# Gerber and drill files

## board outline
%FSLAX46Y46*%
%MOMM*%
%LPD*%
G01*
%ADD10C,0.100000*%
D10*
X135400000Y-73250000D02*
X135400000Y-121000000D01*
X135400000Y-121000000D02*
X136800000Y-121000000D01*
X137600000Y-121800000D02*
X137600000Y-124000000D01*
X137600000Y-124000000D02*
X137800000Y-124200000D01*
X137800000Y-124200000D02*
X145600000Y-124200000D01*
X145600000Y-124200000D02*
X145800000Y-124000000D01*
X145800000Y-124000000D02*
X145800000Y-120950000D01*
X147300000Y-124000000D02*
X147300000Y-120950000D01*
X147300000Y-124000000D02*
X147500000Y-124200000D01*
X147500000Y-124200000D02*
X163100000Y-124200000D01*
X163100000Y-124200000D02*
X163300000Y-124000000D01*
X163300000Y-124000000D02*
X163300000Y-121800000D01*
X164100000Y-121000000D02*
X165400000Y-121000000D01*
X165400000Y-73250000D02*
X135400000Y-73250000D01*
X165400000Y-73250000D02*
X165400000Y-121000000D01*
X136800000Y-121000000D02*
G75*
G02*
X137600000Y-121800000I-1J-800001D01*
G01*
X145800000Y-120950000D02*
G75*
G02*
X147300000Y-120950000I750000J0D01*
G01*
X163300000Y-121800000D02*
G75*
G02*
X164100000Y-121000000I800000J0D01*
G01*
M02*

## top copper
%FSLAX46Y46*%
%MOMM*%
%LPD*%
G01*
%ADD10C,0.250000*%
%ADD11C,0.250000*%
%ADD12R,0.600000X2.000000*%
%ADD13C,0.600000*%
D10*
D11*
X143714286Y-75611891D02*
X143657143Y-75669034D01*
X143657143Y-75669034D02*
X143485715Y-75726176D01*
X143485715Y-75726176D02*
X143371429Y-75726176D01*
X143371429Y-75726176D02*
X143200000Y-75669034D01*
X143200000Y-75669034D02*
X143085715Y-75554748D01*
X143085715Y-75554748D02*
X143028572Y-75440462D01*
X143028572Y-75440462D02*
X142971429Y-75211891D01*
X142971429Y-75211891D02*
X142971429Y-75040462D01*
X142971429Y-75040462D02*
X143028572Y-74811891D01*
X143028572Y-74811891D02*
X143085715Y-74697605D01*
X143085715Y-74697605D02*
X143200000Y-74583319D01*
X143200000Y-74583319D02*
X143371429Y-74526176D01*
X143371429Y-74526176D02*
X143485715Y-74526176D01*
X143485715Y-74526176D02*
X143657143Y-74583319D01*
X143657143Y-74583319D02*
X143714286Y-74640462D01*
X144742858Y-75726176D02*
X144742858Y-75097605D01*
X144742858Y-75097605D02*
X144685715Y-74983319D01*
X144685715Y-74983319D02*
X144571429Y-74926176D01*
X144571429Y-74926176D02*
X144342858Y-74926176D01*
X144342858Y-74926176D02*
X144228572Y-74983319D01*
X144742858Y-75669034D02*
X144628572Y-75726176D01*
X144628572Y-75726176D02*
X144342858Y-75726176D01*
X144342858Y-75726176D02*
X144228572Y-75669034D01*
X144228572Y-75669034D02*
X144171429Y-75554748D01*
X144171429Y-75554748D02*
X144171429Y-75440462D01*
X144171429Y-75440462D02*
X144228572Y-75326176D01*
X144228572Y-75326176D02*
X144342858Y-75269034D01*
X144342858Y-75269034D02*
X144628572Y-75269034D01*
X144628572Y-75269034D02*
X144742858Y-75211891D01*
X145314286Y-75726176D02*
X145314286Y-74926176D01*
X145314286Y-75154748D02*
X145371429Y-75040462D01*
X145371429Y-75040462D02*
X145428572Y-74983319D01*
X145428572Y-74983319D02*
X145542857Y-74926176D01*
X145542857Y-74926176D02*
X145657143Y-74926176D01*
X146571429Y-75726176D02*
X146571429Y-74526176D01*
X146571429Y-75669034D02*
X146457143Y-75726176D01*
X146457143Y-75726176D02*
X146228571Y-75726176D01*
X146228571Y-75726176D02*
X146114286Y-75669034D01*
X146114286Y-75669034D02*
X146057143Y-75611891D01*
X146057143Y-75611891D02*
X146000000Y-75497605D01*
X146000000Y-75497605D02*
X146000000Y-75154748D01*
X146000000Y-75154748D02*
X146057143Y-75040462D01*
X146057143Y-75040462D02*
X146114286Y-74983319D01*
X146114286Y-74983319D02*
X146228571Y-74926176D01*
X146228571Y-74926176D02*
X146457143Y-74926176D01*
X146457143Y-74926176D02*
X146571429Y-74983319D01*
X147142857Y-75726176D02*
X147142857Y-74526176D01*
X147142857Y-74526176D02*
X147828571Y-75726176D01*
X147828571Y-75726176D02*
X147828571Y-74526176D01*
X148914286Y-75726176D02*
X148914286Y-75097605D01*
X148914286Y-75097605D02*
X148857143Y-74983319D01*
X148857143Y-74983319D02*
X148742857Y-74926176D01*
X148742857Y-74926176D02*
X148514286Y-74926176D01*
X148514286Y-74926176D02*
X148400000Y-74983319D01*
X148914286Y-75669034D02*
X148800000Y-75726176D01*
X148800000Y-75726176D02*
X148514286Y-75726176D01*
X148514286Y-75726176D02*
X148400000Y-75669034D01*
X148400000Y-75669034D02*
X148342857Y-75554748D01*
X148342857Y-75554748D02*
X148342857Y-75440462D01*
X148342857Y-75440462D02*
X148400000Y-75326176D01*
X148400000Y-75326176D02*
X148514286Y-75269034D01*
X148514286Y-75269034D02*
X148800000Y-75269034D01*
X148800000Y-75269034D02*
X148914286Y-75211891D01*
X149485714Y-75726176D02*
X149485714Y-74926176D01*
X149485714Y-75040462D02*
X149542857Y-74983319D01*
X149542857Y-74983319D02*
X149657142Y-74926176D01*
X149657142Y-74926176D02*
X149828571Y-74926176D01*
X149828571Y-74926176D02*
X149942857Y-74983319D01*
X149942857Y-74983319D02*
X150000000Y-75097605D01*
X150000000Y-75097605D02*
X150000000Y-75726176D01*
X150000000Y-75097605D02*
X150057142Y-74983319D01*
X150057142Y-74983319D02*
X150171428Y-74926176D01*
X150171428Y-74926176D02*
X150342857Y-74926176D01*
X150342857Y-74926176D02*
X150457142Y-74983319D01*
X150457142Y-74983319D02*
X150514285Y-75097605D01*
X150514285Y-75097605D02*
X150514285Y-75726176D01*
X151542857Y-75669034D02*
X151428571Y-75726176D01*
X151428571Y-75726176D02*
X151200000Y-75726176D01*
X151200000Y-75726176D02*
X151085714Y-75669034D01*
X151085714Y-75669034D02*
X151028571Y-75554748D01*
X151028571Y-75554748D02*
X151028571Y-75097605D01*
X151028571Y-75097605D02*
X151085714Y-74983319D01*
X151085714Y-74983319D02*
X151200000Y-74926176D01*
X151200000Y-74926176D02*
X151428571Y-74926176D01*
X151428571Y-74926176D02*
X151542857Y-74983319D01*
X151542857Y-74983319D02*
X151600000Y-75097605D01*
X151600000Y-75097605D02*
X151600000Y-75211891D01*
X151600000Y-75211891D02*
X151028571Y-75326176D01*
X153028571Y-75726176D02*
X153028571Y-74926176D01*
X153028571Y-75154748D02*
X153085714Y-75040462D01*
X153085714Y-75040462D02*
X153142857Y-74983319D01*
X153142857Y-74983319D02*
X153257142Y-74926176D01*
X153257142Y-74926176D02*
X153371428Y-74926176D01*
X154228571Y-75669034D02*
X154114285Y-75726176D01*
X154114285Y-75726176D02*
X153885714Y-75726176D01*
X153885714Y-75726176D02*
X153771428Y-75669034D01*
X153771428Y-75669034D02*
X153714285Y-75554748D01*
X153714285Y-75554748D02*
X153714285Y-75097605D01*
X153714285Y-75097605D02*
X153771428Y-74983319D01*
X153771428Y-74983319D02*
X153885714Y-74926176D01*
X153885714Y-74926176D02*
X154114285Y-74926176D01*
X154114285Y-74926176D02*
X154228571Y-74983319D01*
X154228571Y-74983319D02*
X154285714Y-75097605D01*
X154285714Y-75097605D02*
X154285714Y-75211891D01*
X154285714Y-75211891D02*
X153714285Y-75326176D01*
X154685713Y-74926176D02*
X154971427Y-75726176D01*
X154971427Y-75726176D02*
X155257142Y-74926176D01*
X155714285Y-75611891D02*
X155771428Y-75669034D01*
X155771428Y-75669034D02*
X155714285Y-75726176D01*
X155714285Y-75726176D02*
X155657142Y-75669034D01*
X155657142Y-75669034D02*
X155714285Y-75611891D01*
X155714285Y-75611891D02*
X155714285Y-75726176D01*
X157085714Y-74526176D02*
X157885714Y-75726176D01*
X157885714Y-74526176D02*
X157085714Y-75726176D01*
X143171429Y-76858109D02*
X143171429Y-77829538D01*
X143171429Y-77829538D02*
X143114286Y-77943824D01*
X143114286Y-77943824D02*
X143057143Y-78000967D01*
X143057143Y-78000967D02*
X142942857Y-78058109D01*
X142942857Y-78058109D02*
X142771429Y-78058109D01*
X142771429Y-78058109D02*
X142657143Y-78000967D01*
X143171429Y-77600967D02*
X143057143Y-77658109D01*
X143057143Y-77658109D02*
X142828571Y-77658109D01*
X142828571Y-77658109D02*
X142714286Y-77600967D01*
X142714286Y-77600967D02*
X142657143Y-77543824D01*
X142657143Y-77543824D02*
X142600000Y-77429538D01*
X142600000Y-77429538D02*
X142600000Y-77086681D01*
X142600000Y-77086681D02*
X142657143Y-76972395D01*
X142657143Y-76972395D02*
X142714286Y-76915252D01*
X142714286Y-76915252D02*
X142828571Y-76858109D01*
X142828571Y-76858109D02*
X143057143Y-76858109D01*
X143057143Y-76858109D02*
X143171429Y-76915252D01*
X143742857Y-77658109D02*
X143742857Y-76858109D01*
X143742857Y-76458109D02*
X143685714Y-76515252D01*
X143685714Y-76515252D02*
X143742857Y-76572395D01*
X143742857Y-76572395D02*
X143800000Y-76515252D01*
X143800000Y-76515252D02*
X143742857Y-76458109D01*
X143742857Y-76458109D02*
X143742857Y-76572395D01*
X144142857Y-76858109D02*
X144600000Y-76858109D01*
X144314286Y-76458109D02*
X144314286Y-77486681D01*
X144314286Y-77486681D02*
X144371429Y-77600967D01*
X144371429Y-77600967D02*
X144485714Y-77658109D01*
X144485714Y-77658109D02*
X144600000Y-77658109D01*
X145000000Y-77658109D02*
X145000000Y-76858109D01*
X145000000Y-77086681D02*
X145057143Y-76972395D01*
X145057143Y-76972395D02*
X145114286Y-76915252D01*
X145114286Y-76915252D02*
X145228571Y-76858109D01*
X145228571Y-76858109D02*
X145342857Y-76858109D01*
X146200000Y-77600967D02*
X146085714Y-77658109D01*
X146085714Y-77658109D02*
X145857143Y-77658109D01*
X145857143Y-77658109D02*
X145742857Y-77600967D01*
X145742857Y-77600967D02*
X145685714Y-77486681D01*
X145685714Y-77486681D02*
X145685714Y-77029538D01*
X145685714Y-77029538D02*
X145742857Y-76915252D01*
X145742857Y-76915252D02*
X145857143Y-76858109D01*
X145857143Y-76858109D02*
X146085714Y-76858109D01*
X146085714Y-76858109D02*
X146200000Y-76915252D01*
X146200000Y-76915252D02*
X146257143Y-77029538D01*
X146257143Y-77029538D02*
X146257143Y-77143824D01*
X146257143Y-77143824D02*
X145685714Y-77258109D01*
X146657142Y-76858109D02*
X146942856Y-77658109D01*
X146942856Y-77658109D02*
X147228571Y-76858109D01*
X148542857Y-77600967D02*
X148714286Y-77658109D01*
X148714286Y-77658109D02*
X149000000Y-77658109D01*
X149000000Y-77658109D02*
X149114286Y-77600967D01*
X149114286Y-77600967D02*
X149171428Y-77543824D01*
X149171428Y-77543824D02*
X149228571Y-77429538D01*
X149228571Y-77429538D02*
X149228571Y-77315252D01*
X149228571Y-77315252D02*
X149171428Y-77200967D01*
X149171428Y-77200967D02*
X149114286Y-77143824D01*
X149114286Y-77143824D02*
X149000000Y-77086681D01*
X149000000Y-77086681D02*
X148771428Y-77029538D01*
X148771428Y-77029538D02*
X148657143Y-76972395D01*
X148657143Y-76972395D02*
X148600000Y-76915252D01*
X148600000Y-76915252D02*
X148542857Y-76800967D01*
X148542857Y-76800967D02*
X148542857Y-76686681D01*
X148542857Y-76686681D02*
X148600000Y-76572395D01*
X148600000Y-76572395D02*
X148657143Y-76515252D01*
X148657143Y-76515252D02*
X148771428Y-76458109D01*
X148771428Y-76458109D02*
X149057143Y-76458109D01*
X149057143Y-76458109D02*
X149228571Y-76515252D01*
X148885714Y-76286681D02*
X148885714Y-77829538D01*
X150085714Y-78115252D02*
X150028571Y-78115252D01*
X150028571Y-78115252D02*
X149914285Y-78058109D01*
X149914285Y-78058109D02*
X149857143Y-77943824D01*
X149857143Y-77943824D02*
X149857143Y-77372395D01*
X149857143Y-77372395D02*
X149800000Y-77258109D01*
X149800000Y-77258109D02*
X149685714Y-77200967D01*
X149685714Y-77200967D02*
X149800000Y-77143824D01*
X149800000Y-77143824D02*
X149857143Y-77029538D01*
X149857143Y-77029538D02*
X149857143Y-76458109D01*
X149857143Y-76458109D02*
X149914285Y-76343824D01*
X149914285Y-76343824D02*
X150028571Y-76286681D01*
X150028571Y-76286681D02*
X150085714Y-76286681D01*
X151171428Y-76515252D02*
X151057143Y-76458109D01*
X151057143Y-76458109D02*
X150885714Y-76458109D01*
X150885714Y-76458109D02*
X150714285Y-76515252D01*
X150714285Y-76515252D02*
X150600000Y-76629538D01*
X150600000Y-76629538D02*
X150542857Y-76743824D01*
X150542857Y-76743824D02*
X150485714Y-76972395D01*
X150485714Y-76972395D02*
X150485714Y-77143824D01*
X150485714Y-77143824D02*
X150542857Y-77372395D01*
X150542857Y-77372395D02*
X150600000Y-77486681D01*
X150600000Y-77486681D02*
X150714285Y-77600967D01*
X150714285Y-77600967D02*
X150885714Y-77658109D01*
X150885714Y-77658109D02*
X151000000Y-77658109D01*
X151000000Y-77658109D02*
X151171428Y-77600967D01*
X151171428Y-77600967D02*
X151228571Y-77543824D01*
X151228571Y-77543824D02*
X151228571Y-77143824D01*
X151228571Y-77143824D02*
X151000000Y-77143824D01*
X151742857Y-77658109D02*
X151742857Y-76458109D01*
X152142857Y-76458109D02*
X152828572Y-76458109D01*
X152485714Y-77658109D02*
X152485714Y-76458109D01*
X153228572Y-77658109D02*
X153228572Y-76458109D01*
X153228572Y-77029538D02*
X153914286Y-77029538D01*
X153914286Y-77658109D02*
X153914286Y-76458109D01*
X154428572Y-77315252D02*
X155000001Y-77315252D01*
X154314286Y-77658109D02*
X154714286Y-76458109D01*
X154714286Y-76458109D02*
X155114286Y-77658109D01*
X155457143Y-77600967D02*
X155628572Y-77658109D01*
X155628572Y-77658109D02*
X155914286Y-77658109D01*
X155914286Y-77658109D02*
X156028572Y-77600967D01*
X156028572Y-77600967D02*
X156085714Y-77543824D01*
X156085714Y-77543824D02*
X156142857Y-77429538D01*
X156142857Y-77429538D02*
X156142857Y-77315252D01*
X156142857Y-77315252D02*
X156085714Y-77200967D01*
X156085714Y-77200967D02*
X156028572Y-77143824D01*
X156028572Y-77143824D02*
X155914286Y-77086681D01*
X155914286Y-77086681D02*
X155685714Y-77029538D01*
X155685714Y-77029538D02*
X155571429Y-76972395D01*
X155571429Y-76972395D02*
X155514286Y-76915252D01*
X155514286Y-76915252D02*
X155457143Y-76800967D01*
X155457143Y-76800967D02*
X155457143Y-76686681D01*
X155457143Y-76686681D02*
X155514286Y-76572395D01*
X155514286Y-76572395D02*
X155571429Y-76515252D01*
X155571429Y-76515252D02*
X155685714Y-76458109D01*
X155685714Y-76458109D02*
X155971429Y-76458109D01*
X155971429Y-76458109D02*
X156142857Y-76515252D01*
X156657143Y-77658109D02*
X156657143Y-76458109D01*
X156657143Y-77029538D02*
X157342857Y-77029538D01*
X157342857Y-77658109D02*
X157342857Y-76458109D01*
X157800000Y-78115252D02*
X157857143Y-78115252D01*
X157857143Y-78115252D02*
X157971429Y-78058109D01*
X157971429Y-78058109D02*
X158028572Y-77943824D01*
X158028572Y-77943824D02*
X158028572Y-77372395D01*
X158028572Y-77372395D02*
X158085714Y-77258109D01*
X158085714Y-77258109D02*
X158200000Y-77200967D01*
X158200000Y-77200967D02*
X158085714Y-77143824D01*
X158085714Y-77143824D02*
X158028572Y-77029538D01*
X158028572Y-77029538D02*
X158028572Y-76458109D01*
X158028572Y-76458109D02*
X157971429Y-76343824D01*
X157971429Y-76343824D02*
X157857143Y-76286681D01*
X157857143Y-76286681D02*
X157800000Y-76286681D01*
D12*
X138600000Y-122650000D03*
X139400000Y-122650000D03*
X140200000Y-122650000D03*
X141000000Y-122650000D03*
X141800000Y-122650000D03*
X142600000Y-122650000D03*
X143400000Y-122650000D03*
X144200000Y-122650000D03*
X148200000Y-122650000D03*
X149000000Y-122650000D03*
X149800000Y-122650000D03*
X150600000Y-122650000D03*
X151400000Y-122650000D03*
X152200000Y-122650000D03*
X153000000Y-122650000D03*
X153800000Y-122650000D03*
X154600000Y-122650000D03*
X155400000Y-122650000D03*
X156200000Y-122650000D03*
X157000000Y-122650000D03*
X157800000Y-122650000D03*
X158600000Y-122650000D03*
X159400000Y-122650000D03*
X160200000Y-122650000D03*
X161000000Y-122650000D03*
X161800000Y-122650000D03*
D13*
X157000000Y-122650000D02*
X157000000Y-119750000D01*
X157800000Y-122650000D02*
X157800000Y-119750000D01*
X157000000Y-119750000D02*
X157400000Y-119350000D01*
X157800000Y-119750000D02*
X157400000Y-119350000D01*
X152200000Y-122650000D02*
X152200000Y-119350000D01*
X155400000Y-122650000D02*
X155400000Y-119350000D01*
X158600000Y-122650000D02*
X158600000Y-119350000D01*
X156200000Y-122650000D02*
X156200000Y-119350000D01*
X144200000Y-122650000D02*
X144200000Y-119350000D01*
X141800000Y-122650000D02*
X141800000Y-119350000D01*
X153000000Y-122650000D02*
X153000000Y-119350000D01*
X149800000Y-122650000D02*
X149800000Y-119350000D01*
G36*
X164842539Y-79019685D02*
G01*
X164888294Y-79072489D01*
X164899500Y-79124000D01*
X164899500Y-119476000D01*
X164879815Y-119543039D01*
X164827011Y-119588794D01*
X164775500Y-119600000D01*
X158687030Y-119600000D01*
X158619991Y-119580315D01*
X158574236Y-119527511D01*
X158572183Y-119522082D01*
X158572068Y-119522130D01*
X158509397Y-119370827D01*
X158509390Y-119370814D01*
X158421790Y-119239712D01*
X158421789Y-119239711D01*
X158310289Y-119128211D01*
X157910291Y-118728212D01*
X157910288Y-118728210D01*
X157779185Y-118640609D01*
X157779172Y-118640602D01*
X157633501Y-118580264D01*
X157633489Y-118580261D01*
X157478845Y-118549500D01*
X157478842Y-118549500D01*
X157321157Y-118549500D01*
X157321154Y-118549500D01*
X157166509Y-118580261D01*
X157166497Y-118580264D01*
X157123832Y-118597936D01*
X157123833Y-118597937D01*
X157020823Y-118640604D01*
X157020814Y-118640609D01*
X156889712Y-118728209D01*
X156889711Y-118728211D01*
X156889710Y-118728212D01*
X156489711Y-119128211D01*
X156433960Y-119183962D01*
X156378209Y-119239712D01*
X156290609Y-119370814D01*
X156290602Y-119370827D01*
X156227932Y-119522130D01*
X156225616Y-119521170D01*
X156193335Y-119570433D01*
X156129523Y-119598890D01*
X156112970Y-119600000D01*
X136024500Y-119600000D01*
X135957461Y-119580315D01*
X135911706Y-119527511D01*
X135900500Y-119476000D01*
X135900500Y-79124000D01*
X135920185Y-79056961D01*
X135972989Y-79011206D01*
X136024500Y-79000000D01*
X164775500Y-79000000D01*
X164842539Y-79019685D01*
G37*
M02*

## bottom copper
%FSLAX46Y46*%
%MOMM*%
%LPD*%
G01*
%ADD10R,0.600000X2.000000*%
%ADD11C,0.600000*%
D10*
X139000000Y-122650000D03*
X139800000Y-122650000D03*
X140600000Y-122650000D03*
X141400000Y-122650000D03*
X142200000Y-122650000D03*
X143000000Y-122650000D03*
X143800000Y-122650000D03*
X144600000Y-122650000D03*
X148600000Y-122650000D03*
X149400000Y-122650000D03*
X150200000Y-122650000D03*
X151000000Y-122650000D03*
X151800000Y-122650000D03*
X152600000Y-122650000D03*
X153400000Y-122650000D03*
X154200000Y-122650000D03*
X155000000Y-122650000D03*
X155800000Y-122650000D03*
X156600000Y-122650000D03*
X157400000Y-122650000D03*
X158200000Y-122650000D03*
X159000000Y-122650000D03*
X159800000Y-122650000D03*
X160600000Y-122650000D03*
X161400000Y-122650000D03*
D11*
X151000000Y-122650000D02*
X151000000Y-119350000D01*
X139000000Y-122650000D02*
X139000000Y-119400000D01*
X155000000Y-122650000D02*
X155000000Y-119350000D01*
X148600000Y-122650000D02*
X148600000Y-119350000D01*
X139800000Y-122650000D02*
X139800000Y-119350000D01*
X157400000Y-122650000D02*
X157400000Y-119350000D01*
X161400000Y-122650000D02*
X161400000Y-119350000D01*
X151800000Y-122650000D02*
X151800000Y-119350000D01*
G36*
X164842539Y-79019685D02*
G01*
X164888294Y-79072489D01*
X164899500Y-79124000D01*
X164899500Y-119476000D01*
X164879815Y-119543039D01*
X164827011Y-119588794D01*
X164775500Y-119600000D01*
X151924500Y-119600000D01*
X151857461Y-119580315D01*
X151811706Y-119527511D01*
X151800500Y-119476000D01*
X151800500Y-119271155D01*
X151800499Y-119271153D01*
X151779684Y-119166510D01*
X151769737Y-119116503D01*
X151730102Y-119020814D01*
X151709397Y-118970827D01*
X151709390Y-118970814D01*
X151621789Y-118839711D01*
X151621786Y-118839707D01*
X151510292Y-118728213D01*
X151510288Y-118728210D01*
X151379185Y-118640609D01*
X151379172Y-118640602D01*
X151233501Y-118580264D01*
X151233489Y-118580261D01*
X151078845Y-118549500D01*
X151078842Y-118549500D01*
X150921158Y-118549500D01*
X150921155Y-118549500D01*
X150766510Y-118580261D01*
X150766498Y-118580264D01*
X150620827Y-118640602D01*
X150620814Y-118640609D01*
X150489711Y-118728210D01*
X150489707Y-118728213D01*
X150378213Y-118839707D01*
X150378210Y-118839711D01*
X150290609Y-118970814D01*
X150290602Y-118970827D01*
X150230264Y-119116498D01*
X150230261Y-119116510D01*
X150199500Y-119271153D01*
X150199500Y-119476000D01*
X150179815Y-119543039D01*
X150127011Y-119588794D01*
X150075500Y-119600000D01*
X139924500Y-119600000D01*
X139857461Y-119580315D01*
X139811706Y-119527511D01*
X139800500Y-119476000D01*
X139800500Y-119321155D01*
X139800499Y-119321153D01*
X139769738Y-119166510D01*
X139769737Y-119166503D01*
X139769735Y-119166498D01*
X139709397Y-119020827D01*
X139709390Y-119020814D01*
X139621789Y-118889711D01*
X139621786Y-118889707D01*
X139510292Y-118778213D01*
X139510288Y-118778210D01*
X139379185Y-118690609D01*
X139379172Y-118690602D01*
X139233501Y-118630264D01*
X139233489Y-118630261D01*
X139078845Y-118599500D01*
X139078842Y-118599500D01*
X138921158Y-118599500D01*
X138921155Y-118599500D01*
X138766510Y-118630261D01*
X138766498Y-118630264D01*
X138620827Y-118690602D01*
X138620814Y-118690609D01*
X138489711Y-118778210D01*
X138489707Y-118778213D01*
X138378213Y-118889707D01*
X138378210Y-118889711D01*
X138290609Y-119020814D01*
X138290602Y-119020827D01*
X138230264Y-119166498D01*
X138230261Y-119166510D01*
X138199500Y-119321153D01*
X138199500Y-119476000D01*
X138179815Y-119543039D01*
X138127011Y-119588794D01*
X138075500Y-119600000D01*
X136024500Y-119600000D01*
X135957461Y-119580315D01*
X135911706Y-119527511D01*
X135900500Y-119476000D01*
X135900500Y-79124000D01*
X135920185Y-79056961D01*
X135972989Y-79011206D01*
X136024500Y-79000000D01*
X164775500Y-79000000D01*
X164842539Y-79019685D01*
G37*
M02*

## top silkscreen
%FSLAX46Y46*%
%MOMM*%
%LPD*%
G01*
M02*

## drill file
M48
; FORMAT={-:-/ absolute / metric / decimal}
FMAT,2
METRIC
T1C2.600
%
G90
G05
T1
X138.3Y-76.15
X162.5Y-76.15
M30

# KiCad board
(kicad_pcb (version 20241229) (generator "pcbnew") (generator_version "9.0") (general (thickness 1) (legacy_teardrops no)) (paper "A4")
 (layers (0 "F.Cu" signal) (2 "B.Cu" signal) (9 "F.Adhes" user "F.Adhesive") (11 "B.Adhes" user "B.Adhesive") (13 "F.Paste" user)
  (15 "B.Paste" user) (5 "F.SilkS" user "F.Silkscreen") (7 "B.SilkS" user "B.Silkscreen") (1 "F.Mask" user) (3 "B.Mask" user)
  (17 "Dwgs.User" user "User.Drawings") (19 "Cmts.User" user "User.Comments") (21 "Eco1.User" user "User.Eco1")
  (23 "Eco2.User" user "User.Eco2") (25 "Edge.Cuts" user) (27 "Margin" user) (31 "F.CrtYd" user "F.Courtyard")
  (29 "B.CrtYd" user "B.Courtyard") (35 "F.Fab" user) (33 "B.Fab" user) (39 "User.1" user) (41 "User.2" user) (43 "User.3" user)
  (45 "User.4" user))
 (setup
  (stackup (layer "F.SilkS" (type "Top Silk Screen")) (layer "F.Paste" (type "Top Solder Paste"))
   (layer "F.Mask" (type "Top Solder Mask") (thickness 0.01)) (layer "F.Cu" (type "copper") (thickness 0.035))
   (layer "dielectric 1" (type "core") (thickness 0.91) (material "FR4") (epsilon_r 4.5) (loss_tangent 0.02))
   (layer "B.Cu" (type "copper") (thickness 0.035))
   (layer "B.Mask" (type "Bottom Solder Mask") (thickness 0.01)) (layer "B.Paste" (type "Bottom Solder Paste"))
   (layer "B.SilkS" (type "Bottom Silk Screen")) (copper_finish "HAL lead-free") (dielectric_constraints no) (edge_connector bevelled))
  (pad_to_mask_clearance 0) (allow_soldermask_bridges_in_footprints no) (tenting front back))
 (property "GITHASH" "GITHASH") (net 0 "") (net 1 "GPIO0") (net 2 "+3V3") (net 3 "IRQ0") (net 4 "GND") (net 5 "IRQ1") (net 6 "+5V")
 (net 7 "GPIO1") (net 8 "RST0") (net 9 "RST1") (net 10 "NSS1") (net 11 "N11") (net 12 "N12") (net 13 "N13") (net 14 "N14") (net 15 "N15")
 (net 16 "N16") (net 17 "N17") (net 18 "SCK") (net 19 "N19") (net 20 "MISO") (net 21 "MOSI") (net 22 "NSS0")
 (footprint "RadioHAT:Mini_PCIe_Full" (layer "F.Cu") (at 137.6 124.2)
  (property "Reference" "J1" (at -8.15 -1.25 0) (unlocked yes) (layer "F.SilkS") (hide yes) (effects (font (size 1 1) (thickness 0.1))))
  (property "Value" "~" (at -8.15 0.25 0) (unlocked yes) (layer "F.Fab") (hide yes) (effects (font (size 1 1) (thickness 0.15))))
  (fp_line (start -2.2 -50.95) (end -2.2 -3.2) (stroke (width 0.1) (type solid)) (layer "Edge.Cuts"))
  (fp_line (start -2.2 -3.2) (end -0.8 -3.2) (stroke (width 0.1) (type solid)) (layer "Edge.Cuts"))
  (fp_line (start 0 -2.4) (end 0 -0.2) (stroke (width 0.1) (type solid)) (layer "Edge.Cuts"))
  (fp_line (start 0 -0.2) (end 0.2 0) (stroke (width 0.1) (type solid)) (layer "Edge.Cuts"))
  (fp_line (start 0.2 0) (end 8 0) (stroke (width 0.1) (type solid)) (layer "Edge.Cuts"))
  (fp_line (start 8 0) (end 8.2 -0.2) (stroke (width 0.1) (type solid)) (layer "Edge.Cuts"))
  (fp_line (start 8.2 -0.2) (end 8.2 -3.25) (stroke (width 0.1) (type solid)) (layer "Edge.Cuts"))
  (fp_line (start 9.7 -0.2) (end 9.7 -3.25) (stroke (width 0.1) (type solid)) (layer "Edge.Cuts"))
  (fp_line (start 9.7 -0.2) (end 9.9 0) (stroke (width 0.1) (type solid)) (layer "Edge.Cuts"))
  (fp_line (start 9.9 0) (end 25.5 0) (stroke (width 0.1) (type solid)) (layer "Edge.Cuts"))
  (fp_line (start 25.5 0) (end 25.7 -0.2) (stroke (width 0.1) (type solid)) (layer "Edge.Cuts"))
  (fp_line (start 25.7 -0.2) (end 25.7 -2.4) (stroke (width 0.1) (type solid)) (layer "Edge.Cuts"))
  (fp_line (start 26.5 -3.2) (end 27.8 -3.2) (stroke (width 0.1) (type solid)) (layer "Edge.Cuts"))
  (fp_line (start 27.8 -50.95) (end -2.2 -50.95) (stroke (width 0.1) (type solid)) (layer "Edge.Cuts"))
  (fp_line (start 27.8 -50.95) (end 27.8 -3.2) (stroke (width 0.1) (type solid)) (layer "Edge.Cuts"))
  (fp_arc (start -0.8 -3.2) (mid -0.234315 -2.965685) (end 0 -2.4) (stroke (width 0.1) (type solid)) (layer "Edge.Cuts"))
  (fp_arc (start 8.2 -3.25) (mid 8.95 -4) (end 9.7 -3.25) (stroke (width 0.1) (type solid)) (layer "Edge.Cuts"))
  (fp_arc (start 25.7 -2.4) (mid 25.934315 -2.965685) (end 26.5 -3.2) (stroke (width 0.1) (type solid)) (layer "Edge.Cuts"))
  (pad "" np_thru_hole circle (at 0.7 -48.05) (size 2.6 2.6) (drill 2.6) (layers "*.Cu" "*.Mask") (thermal_bridge_angle 0))
  (pad "" np_thru_hole circle (at 24.9 -48.05) (size 2.6 2.6) (drill 2.6) (layers "*.Cu" "*.Mask") (thermal_bridge_angle 0))
  (pad "1" smd rect (at 1 -1.55 90) (size 2 0.6) (layers "F.Cu" "F.Mask" "F.Paste") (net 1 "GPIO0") (thermal_bridge_angle 0))
  (pad "2" smd rect (at 1.4 -1.55 90) (size 2 0.6) (layers "B.Cu" "B.Mask" "B.Paste") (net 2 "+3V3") (thermal_bridge_angle 0))
  (pad "3" smd rect (at 1.8 -1.55 90) (size 2 0.6) (layers "F.Cu" "F.Mask" "F.Paste") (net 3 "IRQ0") (thermal_bridge_angle 0))
  (pad "4" smd rect (at 2.2 -1.55 90) (size 2 0.6) (layers "B.Cu" "B.Mask" "B.Paste") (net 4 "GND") (thermal_bridge_angle 0))
  (pad "5" smd rect (at 2.6 -1.55 90) (size 2 0.6) (layers "F.Cu" "F.Mask" "F.Paste") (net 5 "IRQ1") (thermal_bridge_angle 0))
  (pad "6" smd rect (at 3 -1.55 90) (size 2 0.6) (layers "B.Cu" "B.Mask" "B.Paste") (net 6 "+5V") (thermal_bridge_angle 0))
  (pad "7" smd rect (at 3.4 -1.55 90) (size 2 0.6) (layers "F.Cu" "F.Mask" "F.Paste") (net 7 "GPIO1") (thermal_bridge_angle 0))
  (pad "8" smd rect (at 3.8 -1.55 90) (size 2 0.6) (layers "B.Cu" "B.Mask" "B.Paste") (thermal_bridge_angle 0))
  (pad "9" smd rect (at 4.2 -1.55 90) (size 2 0.6) (layers "F.Cu" "F.Mask" "F.Paste") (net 4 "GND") (thermal_bridge_angle 0))
  (pad "10" smd rect (at 4.6 -1.55 90) (size 2 0.6) (layers "B.Cu" "B.Mask" "B.Paste") (thermal_bridge_angle 0))
  (pad "11" smd rect (at 5 -1.55 90) (size 2 0.6) (layers "F.Cu" "F.Mask" "F.Paste") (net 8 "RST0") (thermal_bridge_angle 0))
  (pad "12" smd rect (at 5.4 -1.55 90) (size 2 0.6) (layers "B.Cu" "B.Mask" "B.Paste") (thermal_bridge_angle 0))
  (pad "13" smd rect (at 5.8 -1.55 90) (size 2 0.6) (layers "F.Cu" "F.Mask" "F.Paste") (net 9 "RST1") (thermal_bridge_angle 0))
  (pad "14" smd rect (at 6.2 -1.55 90) (size 2 0.6) (layers "B.Cu" "B.Mask" "B.Paste") (thermal_bridge_angle 0))
  (pad "15" smd rect (at 6.6 -1.55 90) (size 2 0.6) (layers "F.Cu" "F.Mask" "F.Paste") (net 4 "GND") (thermal_bridge_angle 0))
  (pad "16" smd rect (at 7 -1.55 90) (size 2 0.6) (layers "B.Cu" "B.Mask" "B.Paste") (thermal_bridge_angle 0))
  (pad "17" smd rect (at 10.6 -1.55 90) (size 2 0.6) (layers "F.Cu" "F.Mask" "F.Paste") (thermal_bridge_angle 0))
  (pad "18" smd rect (at 11 -1.55 90) (size 2 0.6) (layers "B.Cu" "B.Mask" "B.Paste") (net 4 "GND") (thermal_bridge_angle 0))
  (pad "19" smd rect (at 11.4 -1.55 90) (size 2 0.6) (layers "F.Cu" "F.Mask" "F.Paste") (thermal_bridge_angle 0))
  (pad "20" smd rect (at 11.8 -1.55 90) (size 2 0.6) (layers "B.Cu" "B.Mask" "B.Paste") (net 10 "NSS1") (thermal_bridge_angle 0))
  (pad "21" smd rect (at 12.2 -1.55 90) (size 2 0.6) (layers "F.Cu" "F.Mask" "F.Paste") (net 4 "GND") (thermal_bridge_angle 0))
  (pad "22" smd rect (at 12.6 -1.55 90) (size 2 0.6) (layers "B.Cu" "B.Mask" "B.Paste") (thermal_bridge_angle 0))
  (pad "23" smd rect (at 13 -1.55 90) (size 2 0.6) (layers "F.Cu" "F.Mask" "F.Paste") (thermal_bridge_angle 0))
  (pad "24" smd rect (at 13.4 -1.55 90) (size 2 0.6) (layers "B.Cu" "B.Mask" "B.Paste") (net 2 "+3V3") (thermal_bridge_angle 0))
  (pad "25" smd rect (at 13.8 -1.55 90) (size 2 0.6) (layers "F.Cu" "F.Mask" "F.Paste") (thermal_bridge_angle 0))
  (pad "26" smd rect (at 14.2 -1.55 90) (size 2 0.6) (layers "B.Cu" "B.Mask" "B.Paste") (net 4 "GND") (thermal_bridge_angle 0))
  (pad "27" smd rect (at 14.6 -1.55 90) (size 2 0.6) (layers "F.Cu" "F.Mask" "F.Paste") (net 4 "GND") (thermal_bridge_angle 0))
  (pad "28" smd rect (at 15 -1.55 90) (size 2 0.6) (layers "B.Cu" "B.Mask" "B.Paste") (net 6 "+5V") (thermal_bridge_angle 0))
  (pad "29" smd rect (at 15.4 -1.55 90) (size 2 0.6) (layers "F.Cu" "F.Mask" "F.Paste") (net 4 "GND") (thermal_bridge_angle 0))
  (pad "30" smd rect (at 15.8 -1.55 90) (size 2 0.6) (layers "B.Cu" "B.Mask" "B.Paste") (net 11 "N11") (thermal_bridge_angle 0))
  (pad "31" smd rect (at 16.2 -1.55 90) (size 2 0.6) (layers "F.Cu" "F.Mask" "F.Paste") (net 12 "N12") (thermal_bridge_angle 0))
  (pad "32" smd rect (at 16.6 -1.55 90) (size 2 0.6) (layers "B.Cu" "B.Mask" "B.Paste") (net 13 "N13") (thermal_bridge_angle 0))
  (pad "33" smd rect (at 17 -1.55 90) (size 2 0.6) (layers "F.Cu" "F.Mask" "F.Paste") (thermal_bridge_angle 0))
  (pad "34" smd rect (at 17.4 -1.55 90) (size 2 0.6) (layers "B.Cu" "B.Mask" "B.Paste") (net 4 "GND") (thermal_bridge_angle 0))
  (pad "35" smd rect (at 17.8 -1.55 90) (size 2 0.6) (layers "F.Cu" "F.Mask" "F.Paste") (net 4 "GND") (thermal_bridge_angle 0))
  (pad "36" smd rect (at 18.2 -1.55 90) (size 2 0.6) (layers "B.Cu" "B.Mask" "B.Paste") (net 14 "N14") (thermal_bridge_angle 0))
  (pad "37" smd rect (at 18.6 -1.55 90) (size 2 0.6) (layers "F.Cu" "F.Mask" "F.Paste") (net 4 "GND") (thermal_bridge_angle 0))
  (pad "38" smd rect (at 19 -1.55 90) (size 2 0.6) (layers "B.Cu" "B.Mask" "B.Paste") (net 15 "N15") (thermal_bridge_angle 0))
  (pad "39" smd rect (at 19.4 -1.55 90) (size 2 0.6) (layers "F.Cu" "F.Mask" "F.Paste") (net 2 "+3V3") (thermal_bridge_angle 0))
  (pad "40" smd rect (at 19.8 -1.55 90) (size 2 0.6) (layers "B.Cu" "B.Mask" "B.Paste") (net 4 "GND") (thermal_bridge_angle 0))
  (pad "41" smd rect (at 20.2 -1.55 90) (size 2 0.6) (layers "F.Cu" "F.Mask" "F.Paste") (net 2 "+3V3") (thermal_bridge_angle 0))
  (pad "42" smd rect (at 20.6 -1.55 90) (size 2 0.6) (layers "B.Cu" "B.Mask" "B.Paste") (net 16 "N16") (thermal_bridge_angle 0))
  (pad "43" smd rect (at 21 -1.55 90) (size 2 0.6) (layers "F.Cu" "F.Mask" "F.Paste") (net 4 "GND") (thermal_bridge_angle 0))
  (pad "44" smd rect (at 21.4 -1.55 90) (size 2 0.6) (layers "B.Cu" "B.Mask" "B.Paste") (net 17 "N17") (thermal_bridge_angle 0))
  (pad "45" smd rect (at 21.8 -1.55 90) (size 2 0.6) (layers "F.Cu" "F.Mask" "F.Paste") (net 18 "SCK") (thermal_bridge_angle 0))
  (pad "46" smd rect (at 22.2 -1.55 90) (size 2 0.6) (layers "B.Cu" "B.Mask" "B.Paste") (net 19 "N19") (thermal_bridge_angle 0))
  (pad "47" smd rect (at 22.6 -1.55 90) (size 2 0.6) (layers "F.Cu" "F.Mask" "F.Paste") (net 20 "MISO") (thermal_bridge_angle 0))
  (pad "48" smd rect (at 23 -1.55 90) (size 2 0.6) (layers "B.Cu" "B.Mask" "B.Paste") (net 6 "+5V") (thermal_bridge_angle 0))
  (pad "49" smd rect (at 23.4 -1.55 90) (size 2 0.6) (layers "F.Cu" "F.Mask" "F.Paste") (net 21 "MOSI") (thermal_bridge_angle 0))
  (pad "50" smd rect (at 23.8 -1.55 90) (size 2 0.6) (layers "B.Cu" "B.Mask" "B.Paste") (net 4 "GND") (thermal_bridge_angle 0))
  (pad "51" smd rect (at 24.2 -1.55 90) (size 2 0.6) (layers "F.Cu" "F.Mask" "F.Paste") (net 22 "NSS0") (thermal_bridge_angle 0)))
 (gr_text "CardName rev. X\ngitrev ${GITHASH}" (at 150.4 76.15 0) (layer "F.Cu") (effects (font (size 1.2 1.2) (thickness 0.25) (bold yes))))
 (segment (start 157 122.65) (end 157 119.75) (width 0.6) (layer "F.Cu") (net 2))
 (segment (start 157.8 122.65) (end 157.8 119.75) (width 0.6) (layer "F.Cu") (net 2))
 (segment (start 157 119.75) (end 157.4 119.35) (width 0.6) (layer "F.Cu") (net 2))
 (segment (start 157.8 119.75) (end 157.4 119.35) (width 0.6) (layer "F.Cu") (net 2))
 (segment (start 151 122.65) (end 151 119.35) (width 0.6) (layer "B.Cu") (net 2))
 (segment (start 139 122.65) (end 139 119.4) (width 0.6) (layer "B.Cu") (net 2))
 (segment (start 152.2 122.65) (end 152.2 119.35) (width 0.6) (layer "F.Cu") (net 4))
 (segment (start 155.4 122.65) (end 155.4 119.35) (width 0.6) (layer "F.Cu") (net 4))
 (segment (start 158.6 122.65) (end 158.6 119.35) (width 0.6) (layer "F.Cu") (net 4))
 (segment (start 156.2 122.65) (end 156.2 119.35) (width 0.6) (layer "F.Cu") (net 4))
 (segment (start 144.2 122.65) (end 144.2 119.35) (width 0.6) (layer "F.Cu") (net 4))
 (segment (start 141.8 122.65) (end 141.8 119.35) (width 0.6) (layer "F.Cu") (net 4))
 (segment (start 153 122.65) (end 153 119.35) (width 0.6) (layer "F.Cu") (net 4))
 (segment (start 149.8 122.65) (end 149.8 119.35) (width 0.6) (layer "F.Cu") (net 4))
 (segment (start 155 122.65) (end 155 119.35) (width 0.6) (layer "B.Cu") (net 4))
 (segment (start 148.6 122.65) (end 148.6 119.35) (width 0.6) (layer "B.Cu") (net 4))
 (segment (start 139.8 122.65) (end 139.8 119.35) (width 0.6) (layer "B.Cu") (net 4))
 (segment (start 157.4 122.65) (end 157.4 119.35) (width 0.6) (layer "B.Cu") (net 4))
 (segment (start 161.4 122.65) (end 161.4 119.35) (width 0.6) (layer "B.Cu") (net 4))
 (segment (start 151.8 122.65) (end 151.8 119.35) (width 0.6) (layer "B.Cu") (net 4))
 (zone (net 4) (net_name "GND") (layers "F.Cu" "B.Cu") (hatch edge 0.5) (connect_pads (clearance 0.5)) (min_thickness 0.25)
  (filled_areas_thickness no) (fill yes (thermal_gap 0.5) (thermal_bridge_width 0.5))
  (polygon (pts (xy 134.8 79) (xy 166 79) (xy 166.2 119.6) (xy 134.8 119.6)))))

